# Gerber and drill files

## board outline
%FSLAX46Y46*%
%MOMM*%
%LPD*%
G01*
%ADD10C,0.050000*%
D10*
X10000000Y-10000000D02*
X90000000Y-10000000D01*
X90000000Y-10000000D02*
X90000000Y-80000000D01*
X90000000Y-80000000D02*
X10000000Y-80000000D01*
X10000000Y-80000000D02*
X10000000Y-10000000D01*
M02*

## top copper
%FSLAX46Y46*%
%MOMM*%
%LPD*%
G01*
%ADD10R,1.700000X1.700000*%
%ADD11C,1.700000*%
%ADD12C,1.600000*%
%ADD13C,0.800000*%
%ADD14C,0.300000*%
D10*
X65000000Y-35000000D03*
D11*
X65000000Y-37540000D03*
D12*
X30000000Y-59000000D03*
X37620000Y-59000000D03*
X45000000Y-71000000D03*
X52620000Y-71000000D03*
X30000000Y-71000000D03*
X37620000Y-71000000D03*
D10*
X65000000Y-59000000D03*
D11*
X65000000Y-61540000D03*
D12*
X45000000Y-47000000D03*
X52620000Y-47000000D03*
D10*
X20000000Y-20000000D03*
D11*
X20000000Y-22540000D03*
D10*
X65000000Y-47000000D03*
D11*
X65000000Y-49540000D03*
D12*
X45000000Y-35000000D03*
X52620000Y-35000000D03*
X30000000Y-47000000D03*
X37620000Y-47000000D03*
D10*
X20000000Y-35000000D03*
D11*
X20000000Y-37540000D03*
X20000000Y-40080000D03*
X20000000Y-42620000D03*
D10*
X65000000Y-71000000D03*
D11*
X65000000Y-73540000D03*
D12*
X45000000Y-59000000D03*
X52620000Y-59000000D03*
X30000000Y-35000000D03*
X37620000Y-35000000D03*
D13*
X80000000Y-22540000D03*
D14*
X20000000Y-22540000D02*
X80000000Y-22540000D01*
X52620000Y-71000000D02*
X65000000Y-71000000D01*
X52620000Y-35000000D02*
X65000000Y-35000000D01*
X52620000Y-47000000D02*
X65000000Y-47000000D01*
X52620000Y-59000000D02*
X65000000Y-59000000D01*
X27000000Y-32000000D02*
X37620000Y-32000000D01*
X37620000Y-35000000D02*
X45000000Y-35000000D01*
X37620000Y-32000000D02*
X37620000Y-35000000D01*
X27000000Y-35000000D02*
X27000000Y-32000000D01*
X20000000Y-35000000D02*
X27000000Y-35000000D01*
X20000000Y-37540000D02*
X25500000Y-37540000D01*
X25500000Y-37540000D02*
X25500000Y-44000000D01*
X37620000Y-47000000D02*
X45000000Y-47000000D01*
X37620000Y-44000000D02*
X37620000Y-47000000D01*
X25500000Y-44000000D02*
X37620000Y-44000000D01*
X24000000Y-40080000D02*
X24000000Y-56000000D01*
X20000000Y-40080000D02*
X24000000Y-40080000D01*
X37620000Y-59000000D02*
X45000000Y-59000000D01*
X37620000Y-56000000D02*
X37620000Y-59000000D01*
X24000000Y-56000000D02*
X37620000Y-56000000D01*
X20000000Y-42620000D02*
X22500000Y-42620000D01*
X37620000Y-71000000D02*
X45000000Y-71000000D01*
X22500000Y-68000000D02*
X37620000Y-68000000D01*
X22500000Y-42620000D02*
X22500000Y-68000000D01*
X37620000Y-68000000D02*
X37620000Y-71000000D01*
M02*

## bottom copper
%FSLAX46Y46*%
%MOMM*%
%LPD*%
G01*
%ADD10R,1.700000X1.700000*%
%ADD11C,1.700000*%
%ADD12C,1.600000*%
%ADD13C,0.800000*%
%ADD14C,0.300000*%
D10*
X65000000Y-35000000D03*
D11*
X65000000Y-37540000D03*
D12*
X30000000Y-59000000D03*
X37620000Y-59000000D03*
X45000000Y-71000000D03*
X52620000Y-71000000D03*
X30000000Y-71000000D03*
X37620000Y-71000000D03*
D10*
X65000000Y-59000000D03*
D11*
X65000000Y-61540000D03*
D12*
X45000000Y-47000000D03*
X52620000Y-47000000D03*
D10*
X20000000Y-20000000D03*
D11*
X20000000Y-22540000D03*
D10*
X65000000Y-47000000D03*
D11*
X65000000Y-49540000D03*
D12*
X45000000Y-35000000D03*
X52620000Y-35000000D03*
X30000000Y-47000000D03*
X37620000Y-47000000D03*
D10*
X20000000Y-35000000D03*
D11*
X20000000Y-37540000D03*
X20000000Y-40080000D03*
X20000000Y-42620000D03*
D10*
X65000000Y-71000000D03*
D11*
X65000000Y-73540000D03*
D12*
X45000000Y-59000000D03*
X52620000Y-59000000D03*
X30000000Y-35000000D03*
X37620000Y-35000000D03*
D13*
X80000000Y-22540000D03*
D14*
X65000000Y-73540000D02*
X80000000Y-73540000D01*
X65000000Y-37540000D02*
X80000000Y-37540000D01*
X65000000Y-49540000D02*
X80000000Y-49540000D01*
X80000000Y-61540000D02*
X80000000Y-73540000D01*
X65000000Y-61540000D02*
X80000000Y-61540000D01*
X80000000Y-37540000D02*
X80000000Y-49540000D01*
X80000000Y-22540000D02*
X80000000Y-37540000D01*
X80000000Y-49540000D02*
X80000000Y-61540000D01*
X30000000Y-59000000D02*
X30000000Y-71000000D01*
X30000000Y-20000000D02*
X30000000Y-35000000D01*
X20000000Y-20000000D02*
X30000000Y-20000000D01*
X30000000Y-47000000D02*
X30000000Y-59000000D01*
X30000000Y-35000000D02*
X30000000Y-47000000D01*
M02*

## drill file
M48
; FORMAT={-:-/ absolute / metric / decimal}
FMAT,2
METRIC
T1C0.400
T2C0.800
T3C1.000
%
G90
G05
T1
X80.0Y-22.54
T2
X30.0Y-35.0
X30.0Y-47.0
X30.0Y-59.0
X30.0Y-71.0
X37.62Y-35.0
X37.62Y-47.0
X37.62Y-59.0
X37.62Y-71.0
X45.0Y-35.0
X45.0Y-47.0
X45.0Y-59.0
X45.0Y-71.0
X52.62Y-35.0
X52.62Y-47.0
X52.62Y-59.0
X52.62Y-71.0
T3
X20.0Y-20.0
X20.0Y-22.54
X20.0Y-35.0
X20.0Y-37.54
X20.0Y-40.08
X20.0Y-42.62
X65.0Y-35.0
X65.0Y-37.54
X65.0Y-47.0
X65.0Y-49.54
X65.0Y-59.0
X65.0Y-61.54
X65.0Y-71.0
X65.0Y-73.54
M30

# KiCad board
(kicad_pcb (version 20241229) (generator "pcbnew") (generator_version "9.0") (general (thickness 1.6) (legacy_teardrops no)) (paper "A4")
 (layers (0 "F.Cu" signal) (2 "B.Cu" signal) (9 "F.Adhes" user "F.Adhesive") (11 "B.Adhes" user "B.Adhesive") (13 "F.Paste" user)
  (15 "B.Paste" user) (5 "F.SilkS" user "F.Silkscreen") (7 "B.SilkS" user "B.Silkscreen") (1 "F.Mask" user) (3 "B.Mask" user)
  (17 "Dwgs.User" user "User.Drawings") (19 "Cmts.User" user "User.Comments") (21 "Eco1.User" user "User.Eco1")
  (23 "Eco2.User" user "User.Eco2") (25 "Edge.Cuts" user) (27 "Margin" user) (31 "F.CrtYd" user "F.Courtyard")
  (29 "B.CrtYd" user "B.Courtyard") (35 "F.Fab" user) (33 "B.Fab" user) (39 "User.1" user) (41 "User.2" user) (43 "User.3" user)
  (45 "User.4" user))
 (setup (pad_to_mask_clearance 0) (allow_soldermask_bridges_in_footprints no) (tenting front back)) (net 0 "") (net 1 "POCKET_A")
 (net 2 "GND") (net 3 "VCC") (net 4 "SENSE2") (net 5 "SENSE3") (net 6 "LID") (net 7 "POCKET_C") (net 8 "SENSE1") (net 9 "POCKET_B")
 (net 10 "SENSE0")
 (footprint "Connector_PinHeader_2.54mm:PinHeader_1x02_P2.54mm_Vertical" (layer "F.Cu") (at 65 35)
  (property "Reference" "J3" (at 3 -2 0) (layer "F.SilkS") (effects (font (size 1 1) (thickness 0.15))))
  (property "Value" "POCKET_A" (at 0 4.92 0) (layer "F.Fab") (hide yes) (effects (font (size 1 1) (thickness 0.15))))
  (pad "1" thru_hole rect (at 0 0) (size 1.7 1.7) (drill 1) (layers "*.Cu" "*.Mask") (remove_unused_layers no) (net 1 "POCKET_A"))
  (pad "2" thru_hole circle (at 0 2.54) (size 1.7 1.7) (drill 1) (layers "*.Cu" "*.Mask") (remove_unused_layers no) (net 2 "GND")))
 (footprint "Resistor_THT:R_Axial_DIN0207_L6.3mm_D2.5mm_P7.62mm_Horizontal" (layer "F.Cu") (at 30 59)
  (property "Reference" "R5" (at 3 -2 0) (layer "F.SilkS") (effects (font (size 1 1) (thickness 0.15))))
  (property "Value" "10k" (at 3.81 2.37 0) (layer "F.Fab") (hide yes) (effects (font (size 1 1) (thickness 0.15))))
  (pad "1" thru_hole circle (at 0 0) (size 1.6 1.6) (drill 0.8) (layers "*.Cu" "*.Mask") (remove_unused_layers no) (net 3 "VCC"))
  (pad "2" thru_hole circle (at 7.62 0) (size 1.6 1.6) (drill 0.8) (layers "*.Cu" "*.Mask") (remove_unused_layers no) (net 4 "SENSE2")))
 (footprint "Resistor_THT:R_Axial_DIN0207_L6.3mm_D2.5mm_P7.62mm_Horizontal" (layer "F.Cu") (at 45 71)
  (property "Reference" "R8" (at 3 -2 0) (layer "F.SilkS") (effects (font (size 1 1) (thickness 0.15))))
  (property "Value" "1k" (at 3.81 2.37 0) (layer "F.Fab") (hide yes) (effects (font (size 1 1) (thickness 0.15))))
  (pad "1" thru_hole circle (at 0 0) (size 1.6 1.6) (drill 0.8) (layers "*.Cu" "*.Mask") (remove_unused_layers no) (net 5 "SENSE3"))
  (pad "2" thru_hole circle (at 7.62 0) (size 1.6 1.6) (drill 0.8) (layers "*.Cu" "*.Mask") (remove_unused_layers no) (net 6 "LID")))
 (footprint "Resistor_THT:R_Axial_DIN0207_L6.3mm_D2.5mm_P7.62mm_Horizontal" (layer "F.Cu") (at 30 71)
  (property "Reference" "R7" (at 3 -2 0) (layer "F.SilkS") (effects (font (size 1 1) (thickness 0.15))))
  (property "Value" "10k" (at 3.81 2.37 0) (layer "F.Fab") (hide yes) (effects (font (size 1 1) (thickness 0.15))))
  (pad "1" thru_hole circle (at 0 0) (size 1.6 1.6) (drill 0.8) (layers "*.Cu" "*.Mask") (remove_unused_layers no) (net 3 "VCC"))
  (pad "2" thru_hole circle (at 7.62 0) (size 1.6 1.6) (drill 0.8) (layers "*.Cu" "*.Mask") (remove_unused_layers no) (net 5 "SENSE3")))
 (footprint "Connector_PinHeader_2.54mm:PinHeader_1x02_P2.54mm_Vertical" (layer "F.Cu") (at 65 59)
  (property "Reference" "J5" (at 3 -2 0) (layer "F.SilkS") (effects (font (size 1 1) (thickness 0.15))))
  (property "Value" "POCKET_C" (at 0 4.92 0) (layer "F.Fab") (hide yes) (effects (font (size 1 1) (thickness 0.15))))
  (pad "1" thru_hole rect (at 0 0) (size 1.7 1.7) (drill 1) (layers "*.Cu" "*.Mask") (remove_unused_layers no) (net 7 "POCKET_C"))
  (pad "2" thru_hole circle (at 0 2.54) (size 1.7 1.7) (drill 1) (layers "*.Cu" "*.Mask") (remove_unused_layers no) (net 2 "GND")))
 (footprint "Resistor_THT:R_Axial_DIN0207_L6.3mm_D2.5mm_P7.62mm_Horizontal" (layer "F.Cu") (at 45 47)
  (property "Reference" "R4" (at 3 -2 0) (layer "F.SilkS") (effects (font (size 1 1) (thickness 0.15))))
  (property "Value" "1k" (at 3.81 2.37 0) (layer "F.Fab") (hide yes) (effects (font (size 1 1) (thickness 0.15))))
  (pad "1" thru_hole circle (at 0 0) (size 1.6 1.6) (drill 0.8) (layers "*.Cu" "*.Mask") (remove_unused_layers no) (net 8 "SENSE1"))
  (pad "2" thru_hole circle (at 7.62 0) (size 1.6 1.6) (drill 0.8) (layers "*.Cu" "*.Mask") (remove_unused_layers no) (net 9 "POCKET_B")))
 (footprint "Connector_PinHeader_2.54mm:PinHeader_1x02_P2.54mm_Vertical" (layer "F.Cu") (at 20 20)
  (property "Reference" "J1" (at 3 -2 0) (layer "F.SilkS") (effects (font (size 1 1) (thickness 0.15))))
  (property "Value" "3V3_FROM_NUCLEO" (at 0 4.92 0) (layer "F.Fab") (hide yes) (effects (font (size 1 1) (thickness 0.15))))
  (pad "1" thru_hole rect (at 0 0) (size 1.7 1.7) (drill 1) (layers "*.Cu" "*.Mask") (remove_unused_layers no) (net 3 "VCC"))
  (pad "2" thru_hole circle (at 0 2.54) (size 1.7 1.7) (drill 1) (layers "*.Cu" "*.Mask") (remove_unused_layers no) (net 2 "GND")))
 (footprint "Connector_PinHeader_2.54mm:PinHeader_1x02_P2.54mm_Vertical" (layer "F.Cu") (at 65 47)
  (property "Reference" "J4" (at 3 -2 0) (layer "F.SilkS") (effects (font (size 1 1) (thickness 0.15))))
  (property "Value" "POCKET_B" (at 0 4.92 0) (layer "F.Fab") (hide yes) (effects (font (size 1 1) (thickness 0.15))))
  (pad "1" thru_hole rect (at 0 0) (size 1.7 1.7) (drill 1) (layers "*.Cu" "*.Mask") (remove_unused_layers no) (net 9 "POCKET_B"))
  (pad "2" thru_hole circle (at 0 2.54) (size 1.7 1.7) (drill 1) (layers "*.Cu" "*.Mask") (remove_unused_layers no) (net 2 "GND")))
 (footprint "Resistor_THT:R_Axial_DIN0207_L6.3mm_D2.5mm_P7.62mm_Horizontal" (layer "F.Cu") (at 45 35)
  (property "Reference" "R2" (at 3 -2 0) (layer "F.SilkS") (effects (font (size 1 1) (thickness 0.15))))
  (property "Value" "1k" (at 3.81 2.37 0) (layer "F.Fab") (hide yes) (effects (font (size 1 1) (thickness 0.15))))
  (pad "1" thru_hole circle (at 0 0) (size 1.6 1.6) (drill 0.8) (layers "*.Cu" "*.Mask") (remove_unused_layers no) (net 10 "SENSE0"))
  (pad "2" thru_hole circle (at 7.62 0) (size 1.6 1.6) (drill 0.8) (layers "*.Cu" "*.Mask") (remove_unused_layers no) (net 1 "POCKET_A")))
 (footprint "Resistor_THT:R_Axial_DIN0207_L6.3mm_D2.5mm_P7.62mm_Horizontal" (layer "F.Cu") (at 30 47)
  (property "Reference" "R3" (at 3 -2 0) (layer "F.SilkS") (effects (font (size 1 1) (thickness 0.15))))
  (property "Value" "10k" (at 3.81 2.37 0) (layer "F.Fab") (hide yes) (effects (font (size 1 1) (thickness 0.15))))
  (pad "1" thru_hole circle (at 0 0) (size 1.6 1.6) (drill 0.8) (layers "*.Cu" "*.Mask") (remove_unused_layers no) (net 3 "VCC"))
  (pad "2" thru_hole circle (at 7.62 0) (size 1.6 1.6) (drill 0.8) (layers "*.Cu" "*.Mask") (remove_unused_layers no) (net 8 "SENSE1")))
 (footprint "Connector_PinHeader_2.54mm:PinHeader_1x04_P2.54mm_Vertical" (layer "F.Cu") (at 20 35)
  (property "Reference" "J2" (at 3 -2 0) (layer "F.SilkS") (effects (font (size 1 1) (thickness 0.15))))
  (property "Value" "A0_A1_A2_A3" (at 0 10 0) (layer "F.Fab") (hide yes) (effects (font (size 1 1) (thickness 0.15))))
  (pad "1" thru_hole rect (at 0 0) (size 1.7 1.7) (drill 1) (layers "*.Cu" "*.Mask") (remove_unused_layers no) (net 10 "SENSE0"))
  (pad "2" thru_hole circle (at 0 2.54) (size 1.7 1.7) (drill 1) (layers "*.Cu" "*.Mask") (remove_unused_layers no) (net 8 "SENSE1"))
  (pad "3" thru_hole circle (at 0 5.08) (size 1.7 1.7) (drill 1) (layers "*.Cu" "*.Mask") (remove_unused_layers no) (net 4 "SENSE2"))
  (pad "4" thru_hole circle (at 0 7.62) (size 1.7 1.7) (drill 1) (layers "*.Cu" "*.Mask") (remove_unused_layers no) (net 5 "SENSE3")))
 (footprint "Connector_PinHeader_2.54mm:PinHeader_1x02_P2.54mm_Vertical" (layer "F.Cu") (at 65 71)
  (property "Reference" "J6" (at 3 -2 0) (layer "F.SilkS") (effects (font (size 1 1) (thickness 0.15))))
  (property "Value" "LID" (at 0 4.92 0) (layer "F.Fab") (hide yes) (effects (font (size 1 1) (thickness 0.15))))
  (pad "1" thru_hole rect (at 0 0) (size 1.7 1.7) (drill 1) (layers "*.Cu" "*.Mask") (remove_unused_layers no) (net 6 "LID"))
  (pad "2" thru_hole circle (at 0 2.54) (size 1.7 1.7) (drill 1) (layers "*.Cu" "*.Mask") (remove_unused_layers no) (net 2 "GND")))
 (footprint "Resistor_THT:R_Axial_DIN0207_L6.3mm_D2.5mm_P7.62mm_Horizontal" (layer "F.Cu") (at 45 59)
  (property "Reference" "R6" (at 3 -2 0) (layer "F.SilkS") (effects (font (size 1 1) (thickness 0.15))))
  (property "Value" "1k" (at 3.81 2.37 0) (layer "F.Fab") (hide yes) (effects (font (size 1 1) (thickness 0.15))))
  (pad "1" thru_hole circle (at 0 0) (size 1.6 1.6) (drill 0.8) (layers "*.Cu" "*.Mask") (remove_unused_layers no) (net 4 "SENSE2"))
  (pad "2" thru_hole circle (at 7.62 0) (size 1.6 1.6) (drill 0.8) (layers "*.Cu" "*.Mask") (remove_unused_layers no) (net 7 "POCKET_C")))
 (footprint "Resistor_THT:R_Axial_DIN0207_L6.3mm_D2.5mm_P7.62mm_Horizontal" (layer "F.Cu") (at 30 35)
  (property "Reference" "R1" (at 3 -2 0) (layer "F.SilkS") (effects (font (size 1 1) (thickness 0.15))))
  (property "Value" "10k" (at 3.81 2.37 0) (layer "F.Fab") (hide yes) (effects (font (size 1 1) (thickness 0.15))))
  (pad "1" thru_hole circle (at 0 0) (size 1.6 1.6) (drill 0.8) (layers "*.Cu" "*.Mask") (remove_unused_layers no) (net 3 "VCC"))
  (pad "2" thru_hole circle (at 7.62 0) (size 1.6 1.6) (drill 0.8) (layers "*.Cu" "*.Mask") (remove_unused_layers no) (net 10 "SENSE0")))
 (gr_line (start 10 10) (end 90 10) (stroke (width 0.05) (type default)) (layer "Edge.Cuts"))
 (gr_line (start 90 10) (end 90 80) (stroke (width 0.05) (type default)) (layer "Edge.Cuts"))
 (gr_line (start 90 80) (end 10 80) (stroke (width 0.05) (type default)) (layer "Edge.Cuts"))
 (gr_line (start 10 80) (end 10 10) (stroke (width 0.05) (type default)) (layer "Edge.Cuts"))
 (segment (start 20 22.54) (end 80 22.54) (width 0.3) (layer "F.Cu") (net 2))
 (via (at 80 22.54) (size 0.8) (drill 0.4) (layers "F.Cu" "B.Cu") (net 2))
 (segment (start 65 73.54) (end 80 73.54) (width 0.3) (layer "B.Cu") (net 2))
 (segment (start 65 37.54) (end 80 37.54) (width 0.3) (layer "B.Cu") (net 2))
 (segment (start 65 49.54) (end 80 49.54) (width 0.3) (layer "B.Cu") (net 2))
 (segment (start 80 61.54) (end 80 73.54) (width 0.3) (layer "B.Cu") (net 2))
 (segment (start 65 61.54) (end 80 61.54) (width 0.3) (layer "B.Cu") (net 2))
 (segment (start 80 37.54) (end 80 49.54) (width 0.3) (layer "B.Cu") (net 2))
 (segment (start 80 22.54) (end 80 37.54) (width 0.3) (layer "B.Cu") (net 2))
 (segment (start 80 49.54) (end 80 61.54) (width 0.3) (layer "B.Cu") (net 2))
 (segment (start 52.62 71) (end 65 71) (width 0.3) (layer "F.Cu") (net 6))
 (segment (start 52.62 35) (end 65 35) (width 0.3) (layer "F.Cu") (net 1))
 (segment (start 52.62 47) (end 65 47) (width 0.3) (layer "F.Cu") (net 9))
 (segment (start 52.62 59) (end 65 59) (width 0.3) (layer "F.Cu") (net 7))
 (segment (start 27 32) (end 37.62 32) (width 0.3) (layer "F.Cu") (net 10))
 (segment (start 37.62 35) (end 45 35) (width 0.3) (layer "F.Cu") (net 10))
 (segment (start 37.62 32) (end 37.62 35) (width 0.3) (layer "F.Cu") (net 10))
 (segment (start 27 35) (end 27 32) (width 0.3) (layer "F.Cu") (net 10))
 (segment (start 20 35) (end 27 35) (width 0.3) (layer "F.Cu") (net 10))
 (segment (start 20 37.54) (end 25.5 37.54) (width 0.3) (layer "F.Cu") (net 8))
 (segment (start 25.5 37.54) (end 25.5 44) (width 0.3) (layer "F.Cu") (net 8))
 (segment (start 37.62 47) (end 45 47) (width 0.3) (layer "F.Cu") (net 8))
 (segment (start 37.62 44) (end 37.62 47) (width 0.3) (layer "F.Cu") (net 8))
 (segment (start 25.5 44) (end 37.62 44) (width 0.3) (layer "F.Cu") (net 8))
 (segment (start 24 40.08) (end 24 56) (width 0.3) (layer "F.Cu") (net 4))
 (segment (start 20 40.08) (end 24 40.08) (width 0.3) (layer "F.Cu") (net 4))
 (segment (start 37.62 59) (end 45 59) (width 0.3) (layer "F.Cu") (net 4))
 (segment (start 37.62 56) (end 37.62 59) (width 0.3) (layer "F.Cu") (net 4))
 (segment (start 24 56) (end 37.62 56) (width 0.3) (layer "F.Cu") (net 4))
 (segment (start 20 42.62) (end 22.5 42.62) (width 0.3) (layer "F.Cu") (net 5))
 (segment (start 37.62 71) (end 45 71) (width 0.3) (layer "F.Cu") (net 5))
 (segment (start 22.5 68) (end 37.62 68) (width 0.3) (layer "F.Cu") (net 5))
 (segment (start 22.5 42.62) (end 22.5 68) (width 0.3) (layer "F.Cu") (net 5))
 (segment (start 37.62 68) (end 37.62 71) (width 0.3) (layer "F.Cu") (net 5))
 (segment (start 30 59) (end 30 71) (width 0.3) (layer "B.Cu") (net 3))
 (segment (start 30 20) (end 30 35) (width 0.3) (layer "B.Cu") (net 3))
 (segment (start 20 20) (end 30 20) (width 0.3) (layer "B.Cu") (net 3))
 (segment (start 30 47) (end 30 59) (width 0.3) (layer "B.Cu") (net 3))
 (segment (start 30 35) (end 30 47) (width 0.3) (layer "B.Cu") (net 3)))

